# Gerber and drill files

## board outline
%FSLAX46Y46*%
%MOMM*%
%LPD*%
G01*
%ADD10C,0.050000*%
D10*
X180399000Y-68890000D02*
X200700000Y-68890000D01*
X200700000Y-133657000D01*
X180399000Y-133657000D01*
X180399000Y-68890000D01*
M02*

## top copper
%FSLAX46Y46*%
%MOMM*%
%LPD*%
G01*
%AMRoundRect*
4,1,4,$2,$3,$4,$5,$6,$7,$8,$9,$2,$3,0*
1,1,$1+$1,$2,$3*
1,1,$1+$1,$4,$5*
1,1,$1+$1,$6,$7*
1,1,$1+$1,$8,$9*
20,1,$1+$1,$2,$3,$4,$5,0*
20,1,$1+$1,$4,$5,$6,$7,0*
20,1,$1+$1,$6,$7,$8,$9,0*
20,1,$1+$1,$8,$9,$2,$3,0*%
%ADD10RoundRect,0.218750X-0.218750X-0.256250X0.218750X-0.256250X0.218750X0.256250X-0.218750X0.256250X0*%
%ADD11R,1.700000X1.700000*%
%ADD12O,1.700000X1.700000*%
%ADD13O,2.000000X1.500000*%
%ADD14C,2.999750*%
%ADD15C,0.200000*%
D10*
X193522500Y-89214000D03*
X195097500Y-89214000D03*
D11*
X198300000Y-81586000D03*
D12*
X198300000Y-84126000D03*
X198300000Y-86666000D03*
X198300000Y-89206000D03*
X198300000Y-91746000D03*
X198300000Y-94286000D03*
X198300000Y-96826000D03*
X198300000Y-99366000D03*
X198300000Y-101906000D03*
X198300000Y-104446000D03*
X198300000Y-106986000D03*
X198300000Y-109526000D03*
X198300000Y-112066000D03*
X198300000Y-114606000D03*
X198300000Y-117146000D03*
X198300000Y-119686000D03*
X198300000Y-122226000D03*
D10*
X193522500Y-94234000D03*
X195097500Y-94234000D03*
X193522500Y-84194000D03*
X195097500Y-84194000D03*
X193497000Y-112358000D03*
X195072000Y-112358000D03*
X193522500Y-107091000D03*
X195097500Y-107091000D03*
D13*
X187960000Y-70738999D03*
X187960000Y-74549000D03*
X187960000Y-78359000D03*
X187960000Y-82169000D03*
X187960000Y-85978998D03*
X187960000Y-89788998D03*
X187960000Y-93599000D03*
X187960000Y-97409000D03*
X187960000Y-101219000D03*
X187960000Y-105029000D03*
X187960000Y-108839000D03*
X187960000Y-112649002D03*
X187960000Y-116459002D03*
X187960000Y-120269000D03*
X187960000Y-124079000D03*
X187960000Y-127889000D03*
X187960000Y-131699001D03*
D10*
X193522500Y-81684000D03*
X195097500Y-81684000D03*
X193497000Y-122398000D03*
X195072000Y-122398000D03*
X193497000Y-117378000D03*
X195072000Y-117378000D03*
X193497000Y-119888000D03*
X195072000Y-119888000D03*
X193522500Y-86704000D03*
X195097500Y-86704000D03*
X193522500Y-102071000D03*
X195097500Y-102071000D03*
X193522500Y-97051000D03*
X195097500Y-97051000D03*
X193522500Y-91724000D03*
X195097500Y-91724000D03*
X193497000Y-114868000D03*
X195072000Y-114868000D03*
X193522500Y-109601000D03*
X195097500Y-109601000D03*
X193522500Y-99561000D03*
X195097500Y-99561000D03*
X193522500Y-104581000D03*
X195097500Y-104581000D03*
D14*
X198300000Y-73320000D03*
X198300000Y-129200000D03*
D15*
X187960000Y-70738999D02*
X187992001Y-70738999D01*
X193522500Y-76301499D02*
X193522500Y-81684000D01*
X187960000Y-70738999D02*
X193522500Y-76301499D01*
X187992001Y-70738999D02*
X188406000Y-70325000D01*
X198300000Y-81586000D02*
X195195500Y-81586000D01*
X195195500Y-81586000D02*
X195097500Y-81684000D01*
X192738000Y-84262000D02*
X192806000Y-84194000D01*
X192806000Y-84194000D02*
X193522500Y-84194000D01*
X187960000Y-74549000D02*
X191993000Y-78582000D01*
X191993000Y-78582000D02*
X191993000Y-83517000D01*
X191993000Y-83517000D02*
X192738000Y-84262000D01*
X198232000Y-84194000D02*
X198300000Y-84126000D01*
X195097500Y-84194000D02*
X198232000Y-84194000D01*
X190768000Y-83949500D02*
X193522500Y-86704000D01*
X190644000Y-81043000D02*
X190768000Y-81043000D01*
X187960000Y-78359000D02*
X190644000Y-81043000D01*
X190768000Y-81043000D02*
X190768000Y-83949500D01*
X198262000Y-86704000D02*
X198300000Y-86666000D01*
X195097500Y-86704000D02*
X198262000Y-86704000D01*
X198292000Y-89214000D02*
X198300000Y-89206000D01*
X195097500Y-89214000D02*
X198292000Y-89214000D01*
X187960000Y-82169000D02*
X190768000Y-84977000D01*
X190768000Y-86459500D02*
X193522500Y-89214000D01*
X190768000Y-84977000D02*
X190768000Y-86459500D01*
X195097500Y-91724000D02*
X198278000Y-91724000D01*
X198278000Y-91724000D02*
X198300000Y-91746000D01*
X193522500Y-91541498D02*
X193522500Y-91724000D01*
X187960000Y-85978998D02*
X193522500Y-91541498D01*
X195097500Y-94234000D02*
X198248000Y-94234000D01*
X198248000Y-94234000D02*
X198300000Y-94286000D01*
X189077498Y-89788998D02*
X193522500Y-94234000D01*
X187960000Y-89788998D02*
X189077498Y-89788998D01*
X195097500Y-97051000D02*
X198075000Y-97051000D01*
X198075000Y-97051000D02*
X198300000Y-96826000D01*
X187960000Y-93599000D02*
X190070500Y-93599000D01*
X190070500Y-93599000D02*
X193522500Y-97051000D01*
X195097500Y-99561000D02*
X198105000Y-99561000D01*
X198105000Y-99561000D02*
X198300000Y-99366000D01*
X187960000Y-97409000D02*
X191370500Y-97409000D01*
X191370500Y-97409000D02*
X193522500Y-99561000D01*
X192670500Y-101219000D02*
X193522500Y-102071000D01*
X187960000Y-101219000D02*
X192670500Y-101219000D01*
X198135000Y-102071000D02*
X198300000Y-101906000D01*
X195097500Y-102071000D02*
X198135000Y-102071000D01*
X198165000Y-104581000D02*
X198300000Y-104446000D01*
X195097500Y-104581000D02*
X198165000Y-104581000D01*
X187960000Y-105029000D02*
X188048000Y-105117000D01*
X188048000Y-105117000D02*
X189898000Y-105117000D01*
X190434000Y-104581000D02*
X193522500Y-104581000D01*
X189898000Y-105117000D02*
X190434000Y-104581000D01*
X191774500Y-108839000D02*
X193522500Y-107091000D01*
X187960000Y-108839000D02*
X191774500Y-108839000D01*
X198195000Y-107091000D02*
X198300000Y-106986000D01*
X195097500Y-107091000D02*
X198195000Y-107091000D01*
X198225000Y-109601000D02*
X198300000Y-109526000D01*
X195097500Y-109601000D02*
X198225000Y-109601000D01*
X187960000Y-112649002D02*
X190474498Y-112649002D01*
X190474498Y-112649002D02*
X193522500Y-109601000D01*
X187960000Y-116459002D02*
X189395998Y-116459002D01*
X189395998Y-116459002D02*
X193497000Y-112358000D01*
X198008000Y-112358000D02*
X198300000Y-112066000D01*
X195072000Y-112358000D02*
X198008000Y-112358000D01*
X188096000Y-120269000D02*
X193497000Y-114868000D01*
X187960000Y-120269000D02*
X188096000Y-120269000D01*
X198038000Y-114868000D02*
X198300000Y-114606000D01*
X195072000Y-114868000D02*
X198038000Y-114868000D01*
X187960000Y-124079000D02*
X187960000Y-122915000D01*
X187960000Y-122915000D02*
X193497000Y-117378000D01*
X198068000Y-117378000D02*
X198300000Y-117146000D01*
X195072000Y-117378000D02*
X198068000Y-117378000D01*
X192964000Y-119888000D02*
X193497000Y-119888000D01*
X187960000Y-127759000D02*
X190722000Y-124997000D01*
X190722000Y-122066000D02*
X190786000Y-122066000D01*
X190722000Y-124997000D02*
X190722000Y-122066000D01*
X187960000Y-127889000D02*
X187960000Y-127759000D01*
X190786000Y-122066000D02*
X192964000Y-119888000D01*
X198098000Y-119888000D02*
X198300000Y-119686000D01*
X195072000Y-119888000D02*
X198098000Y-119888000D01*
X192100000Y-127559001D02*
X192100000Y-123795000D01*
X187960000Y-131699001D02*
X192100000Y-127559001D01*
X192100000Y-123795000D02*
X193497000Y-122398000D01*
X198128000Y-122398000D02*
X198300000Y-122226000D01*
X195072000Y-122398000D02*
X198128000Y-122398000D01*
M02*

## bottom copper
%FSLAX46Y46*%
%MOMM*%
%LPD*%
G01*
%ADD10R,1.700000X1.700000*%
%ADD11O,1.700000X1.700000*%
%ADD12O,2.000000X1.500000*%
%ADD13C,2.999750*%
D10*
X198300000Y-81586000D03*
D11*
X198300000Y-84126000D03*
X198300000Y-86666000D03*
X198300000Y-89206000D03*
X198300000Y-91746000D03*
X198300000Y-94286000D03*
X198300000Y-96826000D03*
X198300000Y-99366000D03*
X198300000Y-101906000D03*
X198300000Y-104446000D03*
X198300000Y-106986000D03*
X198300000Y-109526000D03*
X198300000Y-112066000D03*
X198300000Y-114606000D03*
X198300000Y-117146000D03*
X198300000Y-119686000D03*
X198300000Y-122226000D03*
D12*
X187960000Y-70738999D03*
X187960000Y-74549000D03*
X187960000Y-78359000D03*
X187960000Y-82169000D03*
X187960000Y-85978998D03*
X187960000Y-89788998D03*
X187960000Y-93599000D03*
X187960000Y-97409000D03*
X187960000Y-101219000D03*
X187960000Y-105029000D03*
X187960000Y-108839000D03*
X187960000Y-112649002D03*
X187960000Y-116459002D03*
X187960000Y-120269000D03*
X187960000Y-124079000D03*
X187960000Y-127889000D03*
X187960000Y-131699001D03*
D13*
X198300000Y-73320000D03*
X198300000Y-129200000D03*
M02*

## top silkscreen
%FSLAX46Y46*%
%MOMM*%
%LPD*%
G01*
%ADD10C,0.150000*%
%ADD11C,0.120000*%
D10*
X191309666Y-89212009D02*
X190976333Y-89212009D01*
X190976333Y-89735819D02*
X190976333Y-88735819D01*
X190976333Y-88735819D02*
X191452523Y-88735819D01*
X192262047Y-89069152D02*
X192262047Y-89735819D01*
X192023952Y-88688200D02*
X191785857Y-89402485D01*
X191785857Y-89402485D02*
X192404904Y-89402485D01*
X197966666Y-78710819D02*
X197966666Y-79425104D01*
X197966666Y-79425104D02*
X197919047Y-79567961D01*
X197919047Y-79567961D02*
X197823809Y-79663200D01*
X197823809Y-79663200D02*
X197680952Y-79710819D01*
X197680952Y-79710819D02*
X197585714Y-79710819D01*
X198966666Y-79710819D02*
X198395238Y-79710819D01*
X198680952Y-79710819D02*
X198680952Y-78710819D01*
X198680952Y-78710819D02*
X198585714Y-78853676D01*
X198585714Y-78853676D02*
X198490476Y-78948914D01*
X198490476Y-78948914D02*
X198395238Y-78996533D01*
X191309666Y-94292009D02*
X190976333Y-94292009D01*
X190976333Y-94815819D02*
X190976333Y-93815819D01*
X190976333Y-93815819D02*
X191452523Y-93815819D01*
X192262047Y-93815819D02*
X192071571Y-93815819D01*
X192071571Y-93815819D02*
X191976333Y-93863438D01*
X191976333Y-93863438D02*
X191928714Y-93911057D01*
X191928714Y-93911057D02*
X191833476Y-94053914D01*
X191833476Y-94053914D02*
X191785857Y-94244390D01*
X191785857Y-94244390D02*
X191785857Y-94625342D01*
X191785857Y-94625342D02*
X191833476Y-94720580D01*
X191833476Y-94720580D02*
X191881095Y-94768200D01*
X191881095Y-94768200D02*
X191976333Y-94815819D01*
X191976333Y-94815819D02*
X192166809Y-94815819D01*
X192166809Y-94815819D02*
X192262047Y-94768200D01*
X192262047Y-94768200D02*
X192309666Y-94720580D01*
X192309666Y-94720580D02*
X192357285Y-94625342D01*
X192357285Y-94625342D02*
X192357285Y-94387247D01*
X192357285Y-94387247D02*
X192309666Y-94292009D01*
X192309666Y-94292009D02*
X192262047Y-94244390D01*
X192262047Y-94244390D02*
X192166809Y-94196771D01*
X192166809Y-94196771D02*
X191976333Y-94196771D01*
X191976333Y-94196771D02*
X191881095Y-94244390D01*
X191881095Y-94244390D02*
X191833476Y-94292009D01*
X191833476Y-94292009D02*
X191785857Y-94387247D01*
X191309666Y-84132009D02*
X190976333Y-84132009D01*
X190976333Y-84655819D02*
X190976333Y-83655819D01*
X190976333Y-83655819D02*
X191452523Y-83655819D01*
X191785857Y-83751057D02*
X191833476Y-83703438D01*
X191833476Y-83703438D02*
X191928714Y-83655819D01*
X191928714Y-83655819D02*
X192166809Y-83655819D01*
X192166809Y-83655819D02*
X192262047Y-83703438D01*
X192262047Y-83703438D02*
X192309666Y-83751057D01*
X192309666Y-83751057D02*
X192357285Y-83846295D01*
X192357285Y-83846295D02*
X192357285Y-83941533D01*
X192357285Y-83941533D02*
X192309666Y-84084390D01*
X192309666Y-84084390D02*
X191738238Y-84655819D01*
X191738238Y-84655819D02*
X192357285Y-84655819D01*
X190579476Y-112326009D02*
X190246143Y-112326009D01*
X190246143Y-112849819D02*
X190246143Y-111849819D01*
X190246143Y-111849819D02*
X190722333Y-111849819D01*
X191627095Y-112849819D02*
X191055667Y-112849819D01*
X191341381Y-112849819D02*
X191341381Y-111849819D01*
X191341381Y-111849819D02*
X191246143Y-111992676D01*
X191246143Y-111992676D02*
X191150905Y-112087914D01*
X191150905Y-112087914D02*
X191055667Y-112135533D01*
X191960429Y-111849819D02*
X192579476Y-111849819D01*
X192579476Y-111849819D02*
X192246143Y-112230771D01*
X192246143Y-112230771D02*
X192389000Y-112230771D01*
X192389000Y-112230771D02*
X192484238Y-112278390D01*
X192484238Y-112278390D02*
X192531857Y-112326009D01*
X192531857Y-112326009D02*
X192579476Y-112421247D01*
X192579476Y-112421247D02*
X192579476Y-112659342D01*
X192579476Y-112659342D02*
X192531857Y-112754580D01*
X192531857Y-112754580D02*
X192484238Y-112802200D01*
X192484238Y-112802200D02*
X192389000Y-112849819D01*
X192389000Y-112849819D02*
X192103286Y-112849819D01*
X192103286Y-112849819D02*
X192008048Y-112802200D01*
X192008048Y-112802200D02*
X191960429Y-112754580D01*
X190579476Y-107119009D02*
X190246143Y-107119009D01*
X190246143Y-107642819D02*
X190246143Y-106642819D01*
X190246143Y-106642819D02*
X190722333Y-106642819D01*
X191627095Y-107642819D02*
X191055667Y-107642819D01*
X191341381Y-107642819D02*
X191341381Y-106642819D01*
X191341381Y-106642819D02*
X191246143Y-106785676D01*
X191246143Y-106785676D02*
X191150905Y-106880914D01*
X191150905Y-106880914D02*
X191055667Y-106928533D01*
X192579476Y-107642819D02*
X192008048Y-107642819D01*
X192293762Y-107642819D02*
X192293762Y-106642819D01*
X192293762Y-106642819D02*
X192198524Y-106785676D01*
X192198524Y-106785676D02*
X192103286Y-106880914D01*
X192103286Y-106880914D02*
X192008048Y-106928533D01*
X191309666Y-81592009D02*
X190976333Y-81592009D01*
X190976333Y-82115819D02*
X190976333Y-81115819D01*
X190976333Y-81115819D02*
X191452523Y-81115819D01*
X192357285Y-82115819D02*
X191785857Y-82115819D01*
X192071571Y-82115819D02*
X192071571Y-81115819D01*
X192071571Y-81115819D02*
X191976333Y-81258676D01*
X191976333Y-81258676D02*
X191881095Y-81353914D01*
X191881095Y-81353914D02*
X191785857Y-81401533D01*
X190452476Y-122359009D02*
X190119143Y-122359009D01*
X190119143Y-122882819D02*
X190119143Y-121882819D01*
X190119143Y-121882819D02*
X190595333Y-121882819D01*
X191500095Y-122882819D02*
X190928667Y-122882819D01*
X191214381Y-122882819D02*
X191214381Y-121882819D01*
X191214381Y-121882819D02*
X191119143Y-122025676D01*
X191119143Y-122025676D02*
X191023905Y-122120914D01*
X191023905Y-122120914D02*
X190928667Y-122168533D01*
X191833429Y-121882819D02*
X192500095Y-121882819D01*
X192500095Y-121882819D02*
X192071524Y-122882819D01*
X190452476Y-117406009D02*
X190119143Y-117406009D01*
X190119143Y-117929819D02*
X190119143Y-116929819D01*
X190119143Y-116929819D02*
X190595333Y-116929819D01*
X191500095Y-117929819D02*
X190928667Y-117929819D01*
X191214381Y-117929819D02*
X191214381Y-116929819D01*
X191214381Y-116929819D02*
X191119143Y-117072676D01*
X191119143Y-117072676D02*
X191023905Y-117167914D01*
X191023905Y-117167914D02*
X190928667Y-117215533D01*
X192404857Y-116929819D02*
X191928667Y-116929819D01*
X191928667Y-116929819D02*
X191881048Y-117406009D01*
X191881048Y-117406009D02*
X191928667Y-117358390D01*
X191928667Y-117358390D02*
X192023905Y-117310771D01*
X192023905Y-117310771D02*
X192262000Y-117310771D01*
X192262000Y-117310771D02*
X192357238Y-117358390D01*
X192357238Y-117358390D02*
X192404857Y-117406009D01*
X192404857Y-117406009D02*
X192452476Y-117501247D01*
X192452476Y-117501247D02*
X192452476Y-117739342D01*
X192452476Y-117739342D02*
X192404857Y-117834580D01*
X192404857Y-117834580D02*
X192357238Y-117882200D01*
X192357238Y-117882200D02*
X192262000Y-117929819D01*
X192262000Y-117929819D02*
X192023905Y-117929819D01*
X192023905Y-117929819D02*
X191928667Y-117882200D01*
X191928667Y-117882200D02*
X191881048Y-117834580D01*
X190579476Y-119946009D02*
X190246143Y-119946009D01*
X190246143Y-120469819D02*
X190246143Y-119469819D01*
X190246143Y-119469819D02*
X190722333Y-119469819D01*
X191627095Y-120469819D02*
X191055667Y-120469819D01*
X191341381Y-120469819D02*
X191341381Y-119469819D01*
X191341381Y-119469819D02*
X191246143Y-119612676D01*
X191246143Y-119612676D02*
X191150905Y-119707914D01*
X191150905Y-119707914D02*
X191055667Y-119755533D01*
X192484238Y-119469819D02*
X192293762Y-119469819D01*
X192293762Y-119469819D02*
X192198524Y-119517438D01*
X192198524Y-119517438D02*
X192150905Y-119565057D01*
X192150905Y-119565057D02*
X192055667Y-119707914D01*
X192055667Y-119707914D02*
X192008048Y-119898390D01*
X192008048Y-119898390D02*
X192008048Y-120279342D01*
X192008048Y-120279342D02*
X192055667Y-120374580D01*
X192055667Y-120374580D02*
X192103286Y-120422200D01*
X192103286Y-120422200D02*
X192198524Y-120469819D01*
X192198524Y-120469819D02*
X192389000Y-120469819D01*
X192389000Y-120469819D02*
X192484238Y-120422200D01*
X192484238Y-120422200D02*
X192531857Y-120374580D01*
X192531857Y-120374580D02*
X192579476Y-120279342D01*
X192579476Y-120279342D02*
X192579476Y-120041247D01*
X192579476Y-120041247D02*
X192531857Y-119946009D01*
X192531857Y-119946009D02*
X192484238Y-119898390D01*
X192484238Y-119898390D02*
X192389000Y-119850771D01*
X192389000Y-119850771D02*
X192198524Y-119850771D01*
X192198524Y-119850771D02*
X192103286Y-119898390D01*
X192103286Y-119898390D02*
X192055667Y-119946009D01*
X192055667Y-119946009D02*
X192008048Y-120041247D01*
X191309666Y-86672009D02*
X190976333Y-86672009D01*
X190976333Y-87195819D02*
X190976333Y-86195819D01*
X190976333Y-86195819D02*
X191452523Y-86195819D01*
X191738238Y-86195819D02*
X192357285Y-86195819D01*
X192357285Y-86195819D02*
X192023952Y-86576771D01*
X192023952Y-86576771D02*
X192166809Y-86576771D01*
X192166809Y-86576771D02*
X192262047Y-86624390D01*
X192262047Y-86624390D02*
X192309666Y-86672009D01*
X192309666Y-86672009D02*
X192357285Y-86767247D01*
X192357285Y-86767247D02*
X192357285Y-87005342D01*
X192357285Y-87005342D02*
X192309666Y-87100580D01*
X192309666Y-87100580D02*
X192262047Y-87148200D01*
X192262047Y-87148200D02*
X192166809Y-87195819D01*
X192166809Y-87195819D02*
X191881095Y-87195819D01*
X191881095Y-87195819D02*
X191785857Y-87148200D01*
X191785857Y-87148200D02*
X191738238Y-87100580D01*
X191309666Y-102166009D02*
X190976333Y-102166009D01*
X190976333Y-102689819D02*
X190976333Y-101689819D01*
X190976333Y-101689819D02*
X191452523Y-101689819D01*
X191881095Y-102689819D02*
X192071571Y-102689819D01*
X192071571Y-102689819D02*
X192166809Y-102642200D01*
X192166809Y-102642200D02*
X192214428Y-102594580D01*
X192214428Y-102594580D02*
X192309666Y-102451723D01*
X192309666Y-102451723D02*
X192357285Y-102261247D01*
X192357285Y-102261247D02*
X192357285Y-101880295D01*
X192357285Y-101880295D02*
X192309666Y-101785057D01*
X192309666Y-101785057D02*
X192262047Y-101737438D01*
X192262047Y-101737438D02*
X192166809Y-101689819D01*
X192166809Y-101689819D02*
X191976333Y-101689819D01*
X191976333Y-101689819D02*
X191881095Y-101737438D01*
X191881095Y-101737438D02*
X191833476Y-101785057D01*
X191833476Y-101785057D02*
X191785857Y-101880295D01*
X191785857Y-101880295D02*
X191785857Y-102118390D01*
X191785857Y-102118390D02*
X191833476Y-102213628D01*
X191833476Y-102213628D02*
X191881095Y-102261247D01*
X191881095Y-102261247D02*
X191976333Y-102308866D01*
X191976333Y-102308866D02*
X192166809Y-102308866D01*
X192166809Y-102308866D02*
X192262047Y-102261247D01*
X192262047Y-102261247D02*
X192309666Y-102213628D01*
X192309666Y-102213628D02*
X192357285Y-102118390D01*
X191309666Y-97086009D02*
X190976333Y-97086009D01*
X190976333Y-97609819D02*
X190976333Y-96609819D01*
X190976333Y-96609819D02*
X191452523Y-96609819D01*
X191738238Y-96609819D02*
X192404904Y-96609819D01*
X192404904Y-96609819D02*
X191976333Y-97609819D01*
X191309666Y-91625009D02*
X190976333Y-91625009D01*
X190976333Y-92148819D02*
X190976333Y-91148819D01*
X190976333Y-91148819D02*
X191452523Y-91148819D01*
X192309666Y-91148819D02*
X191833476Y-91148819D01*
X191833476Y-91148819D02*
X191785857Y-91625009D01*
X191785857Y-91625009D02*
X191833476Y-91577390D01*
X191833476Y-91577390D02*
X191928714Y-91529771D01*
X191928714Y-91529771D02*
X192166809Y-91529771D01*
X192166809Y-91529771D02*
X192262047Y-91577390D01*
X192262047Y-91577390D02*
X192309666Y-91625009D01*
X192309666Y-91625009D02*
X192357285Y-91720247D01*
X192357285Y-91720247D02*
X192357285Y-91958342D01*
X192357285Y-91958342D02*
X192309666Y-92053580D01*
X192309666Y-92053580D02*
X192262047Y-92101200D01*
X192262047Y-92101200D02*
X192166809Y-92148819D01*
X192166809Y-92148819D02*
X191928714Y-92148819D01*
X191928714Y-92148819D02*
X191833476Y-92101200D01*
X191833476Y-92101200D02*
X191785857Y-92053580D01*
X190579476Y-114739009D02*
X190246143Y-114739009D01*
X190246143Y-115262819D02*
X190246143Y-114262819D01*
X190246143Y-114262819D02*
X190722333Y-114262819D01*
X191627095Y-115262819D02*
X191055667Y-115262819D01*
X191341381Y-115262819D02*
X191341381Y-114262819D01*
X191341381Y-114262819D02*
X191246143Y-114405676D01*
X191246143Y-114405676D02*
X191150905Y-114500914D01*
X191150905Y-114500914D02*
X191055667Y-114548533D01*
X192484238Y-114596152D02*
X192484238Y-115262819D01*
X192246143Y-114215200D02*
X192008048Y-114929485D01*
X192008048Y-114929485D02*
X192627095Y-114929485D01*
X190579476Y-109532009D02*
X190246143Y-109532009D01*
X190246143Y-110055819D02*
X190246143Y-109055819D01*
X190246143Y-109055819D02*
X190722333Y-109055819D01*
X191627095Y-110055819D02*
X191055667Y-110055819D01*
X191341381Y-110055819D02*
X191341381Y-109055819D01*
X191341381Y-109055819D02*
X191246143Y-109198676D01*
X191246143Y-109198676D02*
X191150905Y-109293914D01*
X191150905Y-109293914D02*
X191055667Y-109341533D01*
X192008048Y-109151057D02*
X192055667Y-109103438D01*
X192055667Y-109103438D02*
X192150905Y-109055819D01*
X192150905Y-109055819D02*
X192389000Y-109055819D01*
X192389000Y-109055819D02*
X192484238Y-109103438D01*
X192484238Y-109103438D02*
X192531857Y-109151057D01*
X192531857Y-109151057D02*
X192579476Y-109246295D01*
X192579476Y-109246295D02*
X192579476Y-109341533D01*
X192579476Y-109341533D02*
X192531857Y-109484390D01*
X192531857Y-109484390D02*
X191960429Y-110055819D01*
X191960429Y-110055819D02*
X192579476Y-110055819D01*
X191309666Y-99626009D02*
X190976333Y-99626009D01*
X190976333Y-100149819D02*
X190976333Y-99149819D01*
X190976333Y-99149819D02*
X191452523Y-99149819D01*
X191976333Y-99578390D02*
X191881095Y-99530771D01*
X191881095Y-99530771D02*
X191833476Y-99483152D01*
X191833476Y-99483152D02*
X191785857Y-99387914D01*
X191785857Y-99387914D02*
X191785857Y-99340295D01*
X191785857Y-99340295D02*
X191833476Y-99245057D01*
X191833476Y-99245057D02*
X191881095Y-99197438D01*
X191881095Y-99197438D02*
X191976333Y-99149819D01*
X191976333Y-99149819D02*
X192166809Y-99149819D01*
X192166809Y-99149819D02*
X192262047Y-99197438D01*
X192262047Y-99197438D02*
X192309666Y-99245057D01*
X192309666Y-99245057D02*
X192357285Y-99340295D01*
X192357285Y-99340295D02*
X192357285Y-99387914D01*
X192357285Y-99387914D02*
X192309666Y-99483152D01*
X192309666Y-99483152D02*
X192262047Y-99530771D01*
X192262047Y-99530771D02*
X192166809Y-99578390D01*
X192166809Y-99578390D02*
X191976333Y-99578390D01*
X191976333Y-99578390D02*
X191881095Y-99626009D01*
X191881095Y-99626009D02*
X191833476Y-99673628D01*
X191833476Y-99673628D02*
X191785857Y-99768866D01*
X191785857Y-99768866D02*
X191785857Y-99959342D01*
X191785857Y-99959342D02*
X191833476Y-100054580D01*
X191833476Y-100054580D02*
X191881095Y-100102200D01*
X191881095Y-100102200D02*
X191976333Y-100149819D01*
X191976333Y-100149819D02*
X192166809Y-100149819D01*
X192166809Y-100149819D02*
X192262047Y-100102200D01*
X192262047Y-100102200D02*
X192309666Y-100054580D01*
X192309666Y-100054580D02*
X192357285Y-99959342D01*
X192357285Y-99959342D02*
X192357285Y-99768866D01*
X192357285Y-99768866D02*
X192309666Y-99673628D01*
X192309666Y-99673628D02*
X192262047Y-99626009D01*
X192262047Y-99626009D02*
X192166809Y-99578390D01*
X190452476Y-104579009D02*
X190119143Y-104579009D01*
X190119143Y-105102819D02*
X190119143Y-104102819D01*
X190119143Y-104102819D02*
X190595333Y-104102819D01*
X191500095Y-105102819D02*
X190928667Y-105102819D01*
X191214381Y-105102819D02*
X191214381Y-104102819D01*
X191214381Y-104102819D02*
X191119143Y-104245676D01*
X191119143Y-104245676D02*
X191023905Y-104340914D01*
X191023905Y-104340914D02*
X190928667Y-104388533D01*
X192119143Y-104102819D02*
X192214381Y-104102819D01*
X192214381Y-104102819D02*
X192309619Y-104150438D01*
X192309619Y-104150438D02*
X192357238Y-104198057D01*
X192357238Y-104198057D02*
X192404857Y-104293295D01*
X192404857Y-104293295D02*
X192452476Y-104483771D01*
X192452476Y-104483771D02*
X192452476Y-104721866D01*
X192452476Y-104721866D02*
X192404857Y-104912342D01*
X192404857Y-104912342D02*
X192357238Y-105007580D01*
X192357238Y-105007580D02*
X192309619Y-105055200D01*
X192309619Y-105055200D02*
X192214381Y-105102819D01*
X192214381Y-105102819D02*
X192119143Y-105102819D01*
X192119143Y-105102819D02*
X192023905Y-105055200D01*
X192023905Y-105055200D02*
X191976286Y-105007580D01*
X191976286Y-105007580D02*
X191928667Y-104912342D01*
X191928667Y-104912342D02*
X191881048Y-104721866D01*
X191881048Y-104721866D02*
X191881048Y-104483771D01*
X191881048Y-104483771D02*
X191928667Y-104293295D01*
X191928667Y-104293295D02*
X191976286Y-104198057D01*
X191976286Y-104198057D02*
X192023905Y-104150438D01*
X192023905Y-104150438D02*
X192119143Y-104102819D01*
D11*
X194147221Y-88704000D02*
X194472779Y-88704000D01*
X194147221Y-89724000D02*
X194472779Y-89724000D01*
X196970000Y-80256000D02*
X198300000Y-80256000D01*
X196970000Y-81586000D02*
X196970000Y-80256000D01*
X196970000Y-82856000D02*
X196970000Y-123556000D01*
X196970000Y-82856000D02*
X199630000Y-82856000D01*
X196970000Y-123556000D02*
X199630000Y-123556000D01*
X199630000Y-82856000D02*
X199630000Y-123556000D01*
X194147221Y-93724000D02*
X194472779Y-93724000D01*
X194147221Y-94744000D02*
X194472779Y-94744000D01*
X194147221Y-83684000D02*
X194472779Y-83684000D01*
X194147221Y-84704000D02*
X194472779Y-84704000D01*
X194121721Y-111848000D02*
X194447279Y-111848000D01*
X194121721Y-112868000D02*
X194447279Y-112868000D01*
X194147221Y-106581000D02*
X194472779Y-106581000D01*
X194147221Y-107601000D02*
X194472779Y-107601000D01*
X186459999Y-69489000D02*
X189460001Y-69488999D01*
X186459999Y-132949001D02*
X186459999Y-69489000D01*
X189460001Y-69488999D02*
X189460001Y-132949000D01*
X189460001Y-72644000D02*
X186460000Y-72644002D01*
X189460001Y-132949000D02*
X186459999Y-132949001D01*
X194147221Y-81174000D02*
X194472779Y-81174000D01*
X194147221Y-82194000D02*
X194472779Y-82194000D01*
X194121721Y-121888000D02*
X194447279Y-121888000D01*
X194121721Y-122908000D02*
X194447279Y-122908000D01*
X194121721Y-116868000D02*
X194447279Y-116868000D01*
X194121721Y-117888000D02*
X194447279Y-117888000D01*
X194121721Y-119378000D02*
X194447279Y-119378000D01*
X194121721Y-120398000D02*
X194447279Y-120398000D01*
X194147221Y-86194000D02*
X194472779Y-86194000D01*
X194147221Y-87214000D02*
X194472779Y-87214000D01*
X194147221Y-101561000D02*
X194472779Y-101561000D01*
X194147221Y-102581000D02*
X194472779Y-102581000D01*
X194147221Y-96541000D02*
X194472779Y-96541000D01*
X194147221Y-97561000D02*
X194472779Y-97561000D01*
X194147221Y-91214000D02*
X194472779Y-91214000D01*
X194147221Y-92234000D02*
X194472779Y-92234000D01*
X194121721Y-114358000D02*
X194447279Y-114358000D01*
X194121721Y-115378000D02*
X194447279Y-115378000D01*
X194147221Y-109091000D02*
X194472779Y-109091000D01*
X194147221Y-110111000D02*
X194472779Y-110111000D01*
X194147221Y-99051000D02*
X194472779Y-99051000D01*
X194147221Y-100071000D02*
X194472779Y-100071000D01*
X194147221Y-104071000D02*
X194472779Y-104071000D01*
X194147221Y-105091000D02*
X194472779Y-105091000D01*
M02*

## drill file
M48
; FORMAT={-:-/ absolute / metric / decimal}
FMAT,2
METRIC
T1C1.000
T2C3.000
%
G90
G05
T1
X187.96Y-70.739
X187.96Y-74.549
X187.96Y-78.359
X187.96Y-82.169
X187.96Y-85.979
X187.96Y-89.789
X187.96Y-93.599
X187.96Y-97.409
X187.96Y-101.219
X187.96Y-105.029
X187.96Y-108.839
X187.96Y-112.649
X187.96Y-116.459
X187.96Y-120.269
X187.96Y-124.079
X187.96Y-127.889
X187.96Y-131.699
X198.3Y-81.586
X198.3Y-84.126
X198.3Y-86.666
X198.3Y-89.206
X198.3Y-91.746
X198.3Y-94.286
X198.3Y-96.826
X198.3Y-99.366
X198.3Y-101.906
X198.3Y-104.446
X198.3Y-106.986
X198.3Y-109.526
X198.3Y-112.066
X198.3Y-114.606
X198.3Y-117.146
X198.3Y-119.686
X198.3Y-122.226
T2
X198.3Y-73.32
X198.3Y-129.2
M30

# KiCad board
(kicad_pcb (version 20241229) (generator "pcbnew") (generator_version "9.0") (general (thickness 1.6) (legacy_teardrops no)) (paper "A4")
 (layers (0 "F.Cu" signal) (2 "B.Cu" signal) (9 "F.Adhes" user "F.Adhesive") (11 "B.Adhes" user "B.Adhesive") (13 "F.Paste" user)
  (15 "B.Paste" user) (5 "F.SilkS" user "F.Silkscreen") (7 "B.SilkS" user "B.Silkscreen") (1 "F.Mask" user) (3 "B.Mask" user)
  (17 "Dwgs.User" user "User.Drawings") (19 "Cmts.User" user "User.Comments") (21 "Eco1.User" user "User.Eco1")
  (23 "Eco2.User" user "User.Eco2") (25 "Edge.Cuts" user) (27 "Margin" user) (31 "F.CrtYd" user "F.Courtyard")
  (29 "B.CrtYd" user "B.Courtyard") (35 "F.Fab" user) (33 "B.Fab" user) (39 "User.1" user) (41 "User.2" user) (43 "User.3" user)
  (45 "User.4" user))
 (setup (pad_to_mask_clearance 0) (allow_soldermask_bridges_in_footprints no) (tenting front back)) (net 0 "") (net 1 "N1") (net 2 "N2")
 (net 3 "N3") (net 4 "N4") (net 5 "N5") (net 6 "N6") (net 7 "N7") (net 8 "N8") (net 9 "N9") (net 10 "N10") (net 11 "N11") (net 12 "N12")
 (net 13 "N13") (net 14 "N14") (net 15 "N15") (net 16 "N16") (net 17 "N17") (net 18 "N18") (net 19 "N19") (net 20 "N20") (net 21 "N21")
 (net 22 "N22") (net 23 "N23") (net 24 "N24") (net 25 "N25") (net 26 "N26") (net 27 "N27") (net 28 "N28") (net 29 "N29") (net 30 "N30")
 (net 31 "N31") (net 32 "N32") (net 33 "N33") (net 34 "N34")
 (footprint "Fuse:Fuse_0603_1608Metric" (layer "F.Cu") (at 194.31 89.214)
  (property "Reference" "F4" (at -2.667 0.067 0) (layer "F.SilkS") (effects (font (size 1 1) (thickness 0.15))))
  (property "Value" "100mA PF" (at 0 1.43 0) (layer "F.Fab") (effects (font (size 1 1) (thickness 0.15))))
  (fp_line (start -0.162779 -0.51) (end 0.162779 -0.51) (stroke (width 0.12) (type solid)) (layer "F.SilkS"))
  (fp_line (start -0.162779 0.51) (end 0.162779 0.51) (stroke (width 0.12) (type solid)) (layer "F.SilkS"))
  (pad "1" smd roundrect (at -0.7875 0) (size 0.875 0.95) (layers "F.Cu" "F.Mask" "F.Paste") (roundrect_rratio 0.25) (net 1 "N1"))
  (pad "2" smd roundrect (at 0.7875 0) (size 0.875 0.95) (layers "F.Cu" "F.Mask" "F.Paste") (roundrect_rratio 0.25) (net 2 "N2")))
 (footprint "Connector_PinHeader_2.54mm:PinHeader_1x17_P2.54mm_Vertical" (layer "F.Cu") (at 198.3 81.586)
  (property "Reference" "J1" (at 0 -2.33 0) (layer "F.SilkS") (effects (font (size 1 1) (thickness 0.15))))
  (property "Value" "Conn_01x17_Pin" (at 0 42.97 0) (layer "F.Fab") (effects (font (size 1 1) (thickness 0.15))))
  (fp_line (start -1.33 -1.33) (end 0 -1.33) (stroke (width 0.12) (type solid)) (layer "F.SilkS"))
  (fp_line (start -1.33 0) (end -1.33 -1.33) (stroke (width 0.12) (type solid)) (layer "F.SilkS"))
  (fp_line (start -1.33 1.27) (end -1.33 41.97) (stroke (width 0.12) (type solid)) (layer "F.SilkS"))
  (fp_line (start -1.33 1.27) (end 1.33 1.27) (stroke (width 0.12) (type solid)) (layer "F.SilkS"))
  (fp_line (start -1.33 41.97) (end 1.33 41.97) (stroke (width 0.12) (type solid)) (layer "F.SilkS"))
  (fp_line (start 1.33 1.27) (end 1.33 41.97) (stroke (width 0.12) (type solid)) (layer "F.SilkS"))
  (pad "1" thru_hole rect (at 0 0) (size 1.7 1.7) (drill 1) (layers "*.Cu" "*.Mask") (remove_unused_layers no) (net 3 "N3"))
  (pad "2" thru_hole oval (at 0 2.54) (size 1.7 1.7) (drill 1) (layers "*.Cu" "*.Mask") (remove_unused_layers no) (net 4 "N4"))
  (pad "3" thru_hole oval (at 0 5.08) (size 1.7 1.7) (drill 1) (layers "*.Cu" "*.Mask") (remove_unused_layers no) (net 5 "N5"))
  (pad "4" thru_hole oval (at 0 7.62) (size 1.7 1.7) (drill 1) (layers "*.Cu" "*.Mask") (remove_unused_layers no) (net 2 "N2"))
  (pad "5" thru_hole oval (at 0 10.16) (size 1.7 1.7) (drill 1) (layers "*.Cu" "*.Mask") (remove_unused_layers no) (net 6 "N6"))
  (pad "6" thru_hole oval (at 0 12.7) (size 1.7 1.7) (drill 1) (layers "*.Cu" "*.Mask") (remove_unused_layers no) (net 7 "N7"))
  (pad "7" thru_hole oval (at 0 15.24) (size 1.7 1.7) (drill 1) (layers "*.Cu" "*.Mask") (remove_unused_layers no) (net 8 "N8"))
  (pad "8" thru_hole oval (at 0 17.78) (size 1.7 1.7) (drill 1) (layers "*.Cu" "*.Mask") (remove_unused_layers no) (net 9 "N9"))
  (pad "9" thru_hole oval (at 0 20.32) (size 1.7 1.7) (drill 1) (layers "*.Cu" "*.Mask") (remove_unused_layers no) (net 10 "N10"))
  (pad "10" thru_hole oval (at 0 22.86) (size 1.7 1.7) (drill 1) (layers "*.Cu" "*.Mask") (remove_unused_layers no) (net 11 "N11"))
  (pad "11" thru_hole oval (at 0 25.4) (size 1.7 1.7) (drill 1) (layers "*.Cu" "*.Mask") (remove_unused_layers no) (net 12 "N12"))
  (pad "12" thru_hole oval (at 0 27.94) (size 1.7 1.7) (drill 1) (layers "*.Cu" "*.Mask") (remove_unused_layers no) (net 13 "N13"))
  (pad "13" thru_hole oval (at 0 30.48) (size 1.7 1.7) (drill 1) (layers "*.Cu" "*.Mask") (remove_unused_layers no) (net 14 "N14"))
  (pad "14" thru_hole oval (at 0 33.02) (size 1.7 1.7) (drill 1) (layers "*.Cu" "*.Mask") (remove_unused_layers no) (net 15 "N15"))
  (pad "15" thru_hole oval (at 0 35.56) (size 1.7 1.7) (drill 1) (layers "*.Cu" "*.Mask") (remove_unused_layers no) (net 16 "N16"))
  (pad "16" thru_hole oval (at 0 38.1) (size 1.7 1.7) (drill 1) (layers "*.Cu" "*.Mask") (remove_unused_layers no) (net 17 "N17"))
  (pad "17" thru_hole oval (at 0 40.64) (size 1.7 1.7) (drill 1) (layers "*.Cu" "*.Mask") (remove_unused_layers no) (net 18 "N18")))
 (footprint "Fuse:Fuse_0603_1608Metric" (layer "F.Cu") (at 194.31 94.234)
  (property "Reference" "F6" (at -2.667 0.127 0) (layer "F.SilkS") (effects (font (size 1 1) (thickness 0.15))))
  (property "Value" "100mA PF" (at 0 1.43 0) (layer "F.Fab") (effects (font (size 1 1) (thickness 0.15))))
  (fp_line (start -0.162779 -0.51) (end 0.162779 -0.51) (stroke (width 0.12) (type solid)) (layer "F.SilkS"))
  (fp_line (start -0.162779 0.51) (end 0.162779 0.51) (stroke (width 0.12) (type solid)) (layer "F.SilkS"))
  (pad "1" smd roundrect (at -0.7875 0) (size 0.875 0.95) (layers "F.Cu" "F.Mask" "F.Paste") (roundrect_rratio 0.25) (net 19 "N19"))
  (pad "2" smd roundrect (at 0.7875 0) (size 0.875 0.95) (layers "F.Cu" "F.Mask" "F.Paste") (roundrect_rratio 0.25) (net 7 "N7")))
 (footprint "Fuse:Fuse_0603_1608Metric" (layer "F.Cu") (at 194.31 84.194)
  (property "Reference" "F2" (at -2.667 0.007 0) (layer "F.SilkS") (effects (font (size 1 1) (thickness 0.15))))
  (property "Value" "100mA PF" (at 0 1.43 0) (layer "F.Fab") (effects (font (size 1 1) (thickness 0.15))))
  (fp_line (start -0.162779 -0.51) (end 0.162779 -0.51) (stroke (width 0.12) (type solid)) (layer "F.SilkS"))
  (fp_line (start -0.162779 0.51) (end 0.162779 0.51) (stroke (width 0.12) (type solid)) (layer "F.SilkS"))
  (pad "1" smd roundrect (at -0.7875 0) (size 0.875 0.95) (layers "F.Cu" "F.Mask" "F.Paste") (roundrect_rratio 0.25) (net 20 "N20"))
  (pad "2" smd roundrect (at 0.7875 0) (size 0.875 0.95) (layers "F.Cu" "F.Mask" "F.Paste") (roundrect_rratio 0.25) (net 4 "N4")))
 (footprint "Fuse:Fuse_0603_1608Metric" (layer "F.Cu") (at 194.2845 112.358)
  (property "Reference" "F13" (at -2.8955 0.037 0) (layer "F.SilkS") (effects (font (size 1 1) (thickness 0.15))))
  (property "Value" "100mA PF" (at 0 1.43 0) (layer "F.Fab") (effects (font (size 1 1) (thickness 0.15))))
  (fp_line (start -0.162779 -0.51) (end 0.162779 -0.51) (stroke (width 0.12) (type solid)) (layer "F.SilkS"))
  (fp_line (start -0.162779 0.51) (end 0.162779 0.51) (stroke (width 0.12) (type solid)) (layer "F.SilkS"))
  (pad "1" smd roundrect (at -0.7875 0) (size 0.875 0.95) (layers "F.Cu" "F.Mask" "F.Paste") (roundrect_rratio 0.25) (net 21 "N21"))
  (pad "2" smd roundrect (at 0.7875 0) (size 0.875 0.95) (layers "F.Cu" "F.Mask" "F.Paste") (roundrect_rratio 0.25) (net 14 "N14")))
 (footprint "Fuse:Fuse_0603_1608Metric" (layer "F.Cu") (at 194.31 107.091)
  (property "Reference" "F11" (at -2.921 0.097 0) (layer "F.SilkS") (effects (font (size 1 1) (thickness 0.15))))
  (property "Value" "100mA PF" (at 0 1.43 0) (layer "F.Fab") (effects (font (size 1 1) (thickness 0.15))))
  (fp_line (start -0.162779 -0.51) (end 0.162779 -0.51) (stroke (width 0.12) (type solid)) (layer "F.SilkS"))
  (fp_line (start -0.162779 0.51) (end 0.162779 0.51) (stroke (width 0.12) (type solid)) (layer "F.SilkS"))
  (pad "1" smd roundrect (at -0.7875 0) (size 0.875 0.95) (layers "F.Cu" "F.Mask" "F.Paste") (roundrect_rratio 0.25) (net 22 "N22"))
  (pad "2" smd roundrect (at 0.7875 0) (size 0.875 0.95) (layers "F.Cu" "F.Mask" "F.Paste") (roundrect_rratio 0.25) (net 12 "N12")))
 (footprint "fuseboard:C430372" (layer "F.Cu") (at 187.96 101.219 -90)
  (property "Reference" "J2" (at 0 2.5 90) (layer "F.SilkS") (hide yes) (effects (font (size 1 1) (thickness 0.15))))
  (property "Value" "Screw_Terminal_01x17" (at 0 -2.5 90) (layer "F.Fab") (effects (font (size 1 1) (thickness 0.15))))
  (fp_line (start -31.73 1.500001) (end -31.730001 -1.500001) (stroke (width 0.12) (type default)) (layer "F.SilkS"))
  (fp_line (start 31.730001 1.500001) (end -31.73 1.500001) (stroke (width 0.12) (type default)) (layer "F.SilkS"))
  (fp_line (start -31.730001 -1.500001) (end 31.73 -1.500001) (stroke (width 0.12) (type default)) (layer "F.SilkS"))
  (fp_line (start -28.575 -1.500001) (end -28.574998 1.5) (stroke (width 0.12) (type default)) (layer "F.SilkS"))
  (fp_line (start 31.73 -1.500001) (end 31.730001 1.500001) (stroke (width 0.12) (type default)) (layer "F.SilkS"))
  (pad "1" thru_hole oval (at -30.480001 0 270) (size 1.5 2) (drill 1) (layers "*.Cu" "*.Mask") (remove_unused_layers no) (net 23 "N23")
   (thermal_bridge_angle 45))
  (pad "2" thru_hole oval (at -26.67 0 270) (size 1.5 2) (drill 1) (layers "*.Cu" "*.Mask") (remove_unused_layers no) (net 20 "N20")
   (thermal_bridge_angle 45))
  (pad "3" thru_hole oval (at -22.86 0 270) (size 1.5 2) (drill 1) (layers "*.Cu" "*.Mask") (remove_unused_layers no) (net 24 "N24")
   (thermal_bridge_angle 45))
  (pad "4" thru_hole oval (at -19.05 0 270) (size 1.5 2) (drill 1) (layers "*.Cu" "*.Mask") (remove_unused_layers no) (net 1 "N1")
   (thermal_bridge_angle 45))
  (pad "5" thru_hole oval (at -15.240002 0 270) (size 1.5 2) (drill 1) (layers "*.Cu" "*.Mask") (remove_unused_layers no) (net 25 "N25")
   (thermal_bridge_angle 45))
  (pad "6" thru_hole oval (at -11.430002 0 270) (size 1.5 2) (drill 1) (layers "*.Cu" "*.Mask") (remove_unused_layers no) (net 19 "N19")
   (thermal_bridge_angle 45))
  (pad "7" thru_hole oval (at -7.62 0 270) (size 1.5 2) (drill 1) (layers "*.Cu" "*.Mask") (remove_unused_layers no) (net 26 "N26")
   (thermal_bridge_angle 45))
  (pad "8" thru_hole oval (at -3.81 0 270) (size 1.5 2) (drill 1) (layers "*.Cu" "*.Mask") (remove_unused_layers no) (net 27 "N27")
   (thermal_bridge_angle 45))
  (pad "9" thru_hole oval (at 0 0 270) (size 1.5 2) (drill 1) (layers "*.Cu" "*.Mask") (remove_unused_layers no) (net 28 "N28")
   (thermal_bridge_angle 45))
  (pad "10" thru_hole oval (at 3.81 0 270) (size 1.5 2) (drill 1) (layers "*.Cu" "*.Mask") (remove_unused_layers no) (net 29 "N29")
   (thermal_bridge_angle 45))
  (pad "11" thru_hole oval (at 7.62 0 270) (size 1.5 2) (drill 1) (layers "*.Cu" "*.Mask") (remove_unused_layers no) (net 22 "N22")
   (thermal_bridge_angle 45))
  (pad "12" thru_hole oval (at 11.430002 0 270) (size 1.5 2) (drill 1) (layers "*.Cu" "*.Mask") (remove_unused_layers no) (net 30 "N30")
   (thermal_bridge_angle 45))
  (pad "13" thru_hole oval (at 15.240002 0 270) (size 1.5 2) (drill 1) (layers "*.Cu" "*.Mask") (remove_unused_layers no) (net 21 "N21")
   (thermal_bridge_angle 45))
  (pad "14" thru_hole oval (at 19.05 0 270) (size 1.5 2) (drill 1) (layers "*.Cu" "*.Mask") (remove_unused_layers no) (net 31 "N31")
   (thermal_bridge_angle 45))
  (pad "15" thru_hole oval (at 22.86 0 270) (size 1.5 2) (drill 1) (layers "*.Cu" "*.Mask") (remove_unused_layers no) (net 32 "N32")
   (thermal_bridge_angle 45))
  (pad "16" thru_hole oval (at 26.67 0 270) (size 1.5 2) (drill 1) (layers "*.Cu" "*.Mask") (remove_unused_layers no) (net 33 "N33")
   (thermal_bridge_angle 45))
  (pad "17" thru_hole oval (at 30.480001 0 270) (size 1.5 2) (drill 1) (layers "*.Cu" "*.Mask") (remove_unused_layers no) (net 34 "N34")
   (thermal_bridge_angle 45)))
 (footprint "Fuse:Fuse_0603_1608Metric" (layer "F.Cu") (at 194.31 81.684)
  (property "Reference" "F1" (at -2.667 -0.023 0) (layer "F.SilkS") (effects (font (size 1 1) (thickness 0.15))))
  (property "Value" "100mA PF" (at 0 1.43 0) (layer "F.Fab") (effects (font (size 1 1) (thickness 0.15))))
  (fp_line (start -0.162779 -0.51) (end 0.162779 -0.51) (stroke (width 0.12) (type solid)) (layer "F.SilkS"))
  (fp_line (start -0.162779 0.51) (end 0.162779 0.51) (stroke (width 0.12) (type solid)) (layer "F.SilkS"))
  (pad "1" smd roundrect (at -0.7875 0) (size 0.875 0.95) (layers "F.Cu" "F.Mask" "F.Paste") (roundrect_rratio 0.25) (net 23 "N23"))
  (pad "2" smd roundrect (at 0.7875 0) (size 0.875 0.95) (layers "F.Cu" "F.Mask" "F.Paste") (roundrect_rratio 0.25) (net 3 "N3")))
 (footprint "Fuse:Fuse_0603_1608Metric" (layer "F.Cu") (at 194.2845 122.398)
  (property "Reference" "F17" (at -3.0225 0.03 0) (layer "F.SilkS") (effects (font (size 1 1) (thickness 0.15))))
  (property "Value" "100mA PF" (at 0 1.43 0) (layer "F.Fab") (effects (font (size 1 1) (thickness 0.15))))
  (fp_line (start -0.162779 -0.51) (end 0.162779 -0.51) (stroke (width 0.12) (type solid)) (layer "F.SilkS"))
  (fp_line (start -0.162779 0.51) (end 0.162779 0.51) (stroke (width 0.12) (type solid)) (layer "F.SilkS"))
  (pad "1" smd roundrect (at -0.7875 0) (size 0.875 0.95) (layers "F.Cu" "F.Mask" "F.Paste") (roundrect_rratio 0.25) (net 34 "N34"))
  (pad "2" smd roundrect (at 0.7875 0) (size 0.875 0.95) (layers "F.Cu" "F.Mask" "F.Paste") (roundrect_rratio 0.25) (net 18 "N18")))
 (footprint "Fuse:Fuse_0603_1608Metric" (layer "F.Cu") (at 194.2845 117.378)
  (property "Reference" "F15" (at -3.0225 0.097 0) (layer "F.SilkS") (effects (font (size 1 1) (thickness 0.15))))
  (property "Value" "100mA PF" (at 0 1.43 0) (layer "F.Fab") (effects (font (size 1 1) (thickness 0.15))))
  (fp_line (start -0.162779 -0.51) (end 0.162779 -0.51) (stroke (width 0.12) (type solid)) (layer "F.SilkS"))
  (fp_line (start -0.162779 0.51) (end 0.162779 0.51) (stroke (width 0.12) (type solid)) (layer "F.SilkS"))
  (pad "1" smd roundrect (at -0.7875 0) (size 0.875 0.95) (layers "F.Cu" "F.Mask" "F.Paste") (roundrect_rratio 0.25) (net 32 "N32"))
  (pad "2" smd roundrect (at 0.7875 0) (size 0.875 0.95) (layers "F.Cu" "F.Mask" "F.Paste") (roundrect_rratio 0.25) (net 16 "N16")))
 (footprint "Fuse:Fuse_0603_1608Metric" (layer "F.Cu") (at 194.2845 119.888)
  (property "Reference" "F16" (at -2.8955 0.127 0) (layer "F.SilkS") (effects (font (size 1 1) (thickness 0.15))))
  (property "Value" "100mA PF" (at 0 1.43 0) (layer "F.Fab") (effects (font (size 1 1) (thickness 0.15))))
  (fp_line (start -0.162779 -0.51) (end 0.162779 -0.51) (stroke (width 0.12) (type solid)) (layer "F.SilkS"))
  (fp_line (start -0.162779 0.51) (end 0.162779 0.51) (stroke (width 0.12) (type solid)) (layer "F.SilkS"))
  (pad "1" smd roundrect (at -0.7875 0) (size 0.875 0.95) (layers "F.Cu" "F.Mask" "F.Paste") (roundrect_rratio 0.25) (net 33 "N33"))
  (pad "2" smd roundrect (at 0.7875 0) (size 0.875 0.95) (layers "F.Cu" "F.Mask" "F.Paste") (roundrect_rratio 0.25) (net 17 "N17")))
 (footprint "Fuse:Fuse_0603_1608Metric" (layer "F.Cu") (at 194.31 86.704)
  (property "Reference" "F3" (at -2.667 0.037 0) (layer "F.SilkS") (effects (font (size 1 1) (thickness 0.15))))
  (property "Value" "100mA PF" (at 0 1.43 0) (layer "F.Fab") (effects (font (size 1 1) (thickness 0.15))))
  (fp_line (start -0.162779 -0.51) (end 0.162779 -0.51) (stroke (width 0.12) (type solid)) (layer "F.SilkS"))
  (fp_line (start -0.162779 0.51) (end 0.162779 0.51) (stroke (width 0.12) (type solid)) (layer "F.SilkS"))
  (pad "1" smd roundrect (at -0.7875 0) (size 0.875 0.95) (layers "F.Cu" "F.Mask" "F.Paste") (roundrect_rratio 0.25) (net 24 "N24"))
  (pad "2" smd roundrect (at 0.7875 0) (size 0.875 0.95) (layers "F.Cu" "F.Mask" "F.Paste") (roundrect_rratio 0.25) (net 5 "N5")))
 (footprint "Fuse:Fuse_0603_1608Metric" (layer "F.Cu") (at 194.31 102.071)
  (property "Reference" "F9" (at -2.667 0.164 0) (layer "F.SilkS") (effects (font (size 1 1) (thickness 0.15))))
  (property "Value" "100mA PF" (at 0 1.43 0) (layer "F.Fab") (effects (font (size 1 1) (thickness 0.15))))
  (fp_line (start -0.162779 -0.51) (end 0.162779 -0.51) (stroke (width 0.12) (type solid)) (layer "F.SilkS"))
  (fp_line (start -0.162779 0.51) (end 0.162779 0.51) (stroke (width 0.12) (type solid)) (layer "F.SilkS"))
  (pad "1" smd roundrect (at -0.7875 0) (size 0.875 0.95) (layers "F.Cu" "F.Mask" "F.Paste") (roundrect_rratio 0.25) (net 28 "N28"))
  (pad "2" smd roundrect (at 0.7875 0) (size 0.875 0.95) (layers "F.Cu" "F.Mask" "F.Paste") (roundrect_rratio 0.25) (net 10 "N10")))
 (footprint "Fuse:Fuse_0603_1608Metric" (layer "F.Cu") (at 194.31 97.051)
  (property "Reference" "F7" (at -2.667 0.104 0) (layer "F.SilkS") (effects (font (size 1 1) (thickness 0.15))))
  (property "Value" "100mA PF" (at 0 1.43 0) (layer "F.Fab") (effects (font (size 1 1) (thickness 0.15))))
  (fp_line (start -0.162779 -0.51) (end 0.162779 -0.51) (stroke (width 0.12) (type solid)) (layer "F.SilkS"))
  (fp_line (start -0.162779 0.51) (end 0.162779 0.51) (stroke (width 0.12) (type solid)) (layer "F.SilkS"))
  (pad "1" smd roundrect (at -0.7875 0) (size 0.875 0.95) (layers "F.Cu" "F.Mask" "F.Paste") (roundrect_rratio 0.25) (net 26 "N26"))
  (pad "2" smd roundrect (at 0.7875 0) (size 0.875 0.95) (layers "F.Cu" "F.Mask" "F.Paste") (roundrect_rratio 0.25) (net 8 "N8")))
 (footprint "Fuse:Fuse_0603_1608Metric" (layer "F.Cu") (at 194.31 91.724)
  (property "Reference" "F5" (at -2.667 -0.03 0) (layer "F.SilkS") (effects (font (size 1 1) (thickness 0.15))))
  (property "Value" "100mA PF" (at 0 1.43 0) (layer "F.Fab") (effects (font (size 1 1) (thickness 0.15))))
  (fp_line (start -0.162779 -0.51) (end 0.162779 -0.51) (stroke (width 0.12) (type solid)) (layer "F.SilkS"))
  (fp_line (start -0.162779 0.51) (end 0.162779 0.51) (stroke (width 0.12) (type solid)) (layer "F.SilkS"))
  (pad "1" smd roundrect (at -0.7875 0) (size 0.875 0.95) (layers "F.Cu" "F.Mask" "F.Paste") (roundrect_rratio 0.25) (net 25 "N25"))
  (pad "2" smd roundrect (at 0.7875 0) (size 0.875 0.95) (layers "F.Cu" "F.Mask" "F.Paste") (roundrect_rratio 0.25) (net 6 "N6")))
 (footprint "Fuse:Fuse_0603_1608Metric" (layer "F.Cu") (at 194.2845 114.868)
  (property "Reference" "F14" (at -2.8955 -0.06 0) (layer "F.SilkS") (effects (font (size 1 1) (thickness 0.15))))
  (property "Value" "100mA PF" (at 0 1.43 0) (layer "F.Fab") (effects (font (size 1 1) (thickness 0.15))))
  (fp_line (start -0.162779 -0.51) (end 0.162779 -0.51) (stroke (width 0.12) (type solid)) (layer "F.SilkS"))
  (fp_line (start -0.162779 0.51) (end 0.162779 0.51) (stroke (width 0.12) (type solid)) (layer "F.SilkS"))
  (pad "1" smd roundrect (at -0.7875 0) (size 0.875 0.95) (layers "F.Cu" "F.Mask" "F.Paste") (roundrect_rratio 0.25) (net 31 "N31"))
  (pad "2" smd roundrect (at 0.7875 0) (size 0.875 0.95) (layers "F.Cu" "F.Mask" "F.Paste") (roundrect_rratio 0.25) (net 15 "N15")))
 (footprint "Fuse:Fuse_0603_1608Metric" (layer "F.Cu") (at 194.31 109.601)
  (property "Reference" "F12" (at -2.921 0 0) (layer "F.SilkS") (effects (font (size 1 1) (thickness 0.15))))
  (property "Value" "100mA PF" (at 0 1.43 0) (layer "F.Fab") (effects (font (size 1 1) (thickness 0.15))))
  (fp_line (start -0.162779 -0.51) (end 0.162779 -0.51) (stroke (width 0.12) (type solid)) (layer "F.SilkS"))
  (fp_line (start -0.162779 0.51) (end 0.162779 0.51) (stroke (width 0.12) (type solid)) (layer "F.SilkS"))
  (pad "1" smd roundrect (at -0.7875 0) (size 0.875 0.95) (layers "F.Cu" "F.Mask" "F.Paste") (roundrect_rratio 0.25) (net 30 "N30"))
  (pad "2" smd roundrect (at 0.7875 0) (size 0.875 0.95) (layers "F.Cu" "F.Mask" "F.Paste") (roundrect_rratio 0.25) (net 13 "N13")))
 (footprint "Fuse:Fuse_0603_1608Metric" (layer "F.Cu") (at 194.31 99.561)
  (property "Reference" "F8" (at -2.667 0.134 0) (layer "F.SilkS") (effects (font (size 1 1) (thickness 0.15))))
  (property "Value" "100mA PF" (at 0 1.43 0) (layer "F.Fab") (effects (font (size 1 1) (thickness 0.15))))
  (fp_line (start -0.162779 -0.51) (end 0.162779 -0.51) (stroke (width 0.12) (type solid)) (layer "F.SilkS"))
  (fp_line (start -0.162779 0.51) (end 0.162779 0.51) (stroke (width 0.12) (type solid)) (layer "F.SilkS"))
  (pad "1" smd roundrect (at -0.7875 0) (size 0.875 0.95) (layers "F.Cu" "F.Mask" "F.Paste") (roundrect_rratio 0.25) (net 27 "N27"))
  (pad "2" smd roundrect (at 0.7875 0) (size 0.875 0.95) (layers "F.Cu" "F.Mask" "F.Paste") (roundrect_rratio 0.25) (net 9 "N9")))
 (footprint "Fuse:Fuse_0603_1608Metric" (layer "F.Cu") (at 194.31 104.581)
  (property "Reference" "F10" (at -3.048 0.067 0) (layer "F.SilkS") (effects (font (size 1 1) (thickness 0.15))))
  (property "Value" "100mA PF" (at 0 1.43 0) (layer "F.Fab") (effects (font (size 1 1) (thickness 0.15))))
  (fp_line (start -0.162779 -0.51) (end 0.162779 -0.51) (stroke (width 0.12) (type solid)) (layer "F.SilkS"))
  (fp_line (start -0.162779 0.51) (end 0.162779 0.51) (stroke (width 0.12) (type solid)) (layer "F.SilkS"))
  (pad "1" smd roundrect (at -0.7875 0) (size 0.875 0.95) (layers "F.Cu" "F.Mask" "F.Paste") (roundrect_rratio 0.25) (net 29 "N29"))
  (pad "2" smd roundrect (at 0.7875 0) (size 0.875 0.95) (layers "F.Cu" "F.Mask" "F.Paste") (roundrect_rratio 0.25) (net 11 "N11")))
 (gr_rect (start 180.399 68.89) (end 200.7 133.657) (stroke (width 0.05) (type default)) (fill no) (layer "Edge.Cuts"))
 (via (at 198.3 73.32) (size 2.99975) (drill 2.99974) (layers "F.Cu" "B.Cu") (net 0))
 (via (at 198.3 129.2) (size 2.99975) (drill 2.99974) (layers "F.Cu" "B.Cu") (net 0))
 (segment (start 187.96 70.738999) (end 187.992001 70.738999) (width 0.2) (layer "F.Cu") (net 23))
 (segment (start 193.5225 76.301499) (end 193.5225 81.684) (width 0.2) (layer "F.Cu") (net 23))
 (segment (start 187.96 70.738999) (end 193.5225 76.301499) (width 0.2) (layer "F.Cu") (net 23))
 (segment (start 187.992001 70.738999) (end 188.406 70.325) (width 0.2) (layer "F.Cu") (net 23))
 (segment (start 198.3 81.586) (end 195.1955 81.586) (width 0.2) (layer "F.Cu") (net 3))
 (segment (start 195.1955 81.586) (end 195.0975 81.684) (width 0.2) (layer "F.Cu") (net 3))
 (segment (start 192.738 84.262) (end 192.806 84.194) (width 0.2) (layer "F.Cu") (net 20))
 (segment (start 192.806 84.194) (end 193.5225 84.194) (width 0.2) (layer "F.Cu") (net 20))
 (segment (start 187.96 74.549) (end 191.993 78.582) (width 0.2) (layer "F.Cu") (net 20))
 (segment (start 191.993 78.582) (end 191.993 83.517) (width 0.2) (layer "F.Cu") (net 20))
 (segment (start 191.993 83.517) (end 192.738 84.262) (width 0.2) (layer "F.Cu") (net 20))
 (segment (start 198.232 84.194) (end 198.3 84.126) (width 0.2) (layer "F.Cu") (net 4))
 (segment (start 195.0975 84.194) (end 198.232 84.194) (width 0.2) (layer "F.Cu") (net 4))
 (segment (start 190.768 83.9495) (end 193.5225 86.704) (width 0.2) (layer "F.Cu") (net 24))
 (segment (start 190.644 81.043) (end 190.768 81.043) (width 0.2) (layer "F.Cu") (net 24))
 (segment (start 187.96 78.359) (end 190.644 81.043) (width 0.2) (layer "F.Cu") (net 24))
 (segment (start 190.768 81.043) (end 190.768 83.9495) (width 0.2) (layer "F.Cu") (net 24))
 (segment (start 198.262 86.704) (end 198.3 86.666) (width 0.2) (layer "F.Cu") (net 5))
 (segment (start 195.0975 86.704) (end 198.262 86.704) (width 0.2) (layer "F.Cu") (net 5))
 (segment (start 198.292 89.214) (end 198.3 89.206) (width 0.2) (layer "F.Cu") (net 2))
 (segment (start 195.0975 89.214) (end 198.292 89.214) (width 0.2) (layer "F.Cu") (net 2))
 (segment (start 187.96 82.169) (end 190.768 84.977) (width 0.2) (layer "F.Cu") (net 1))
 (segment (start 190.768 86.4595) (end 193.5225 89.214) (width 0.2) (layer "F.Cu") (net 1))
 (segment (start 190.768 84.977) (end 190.768 86.4595) (width 0.2) (layer "F.Cu") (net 1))
 (segment (start 195.0975 91.724) (end 198.278 91.724) (width 0.2) (layer "F.Cu") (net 6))
 (segment (start 198.278 91.724) (end 198.3 91.746) (width 0.2) (layer "F.Cu") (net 6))
 (segment (start 193.5225 91.541498) (end 193.5225 91.724) (width 0.2) (layer "F.Cu") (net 25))
 (segment (start 187.96 85.978998) (end 193.5225 91.541498) (width 0.2) (layer "F.Cu") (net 25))
 (segment (start 195.0975 94.234) (end 198.248 94.234) (width 0.2) (layer "F.Cu") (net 7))
 (segment (start 198.248 94.234) (end 198.3 94.286) (width 0.2) (layer "F.Cu") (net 7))
 (segment (start 189.077498 89.788998) (end 193.5225 94.234) (width 0.2) (layer "F.Cu") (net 19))
 (segment (start 187.96 89.788998) (end 189.077498 89.788998) (width 0.2) (layer "F.Cu") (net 19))
 (segment (start 195.0975 97.051) (end 198.075 97.051) (width 0.2) (layer "F.Cu") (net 8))
 (segment (start 198.075 97.051) (end 198.3 96.826) (width 0.2) (layer "F.Cu") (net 8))
 (segment (start 187.96 93.599) (end 190.0705 93.599) (width 0.2) (layer "F.Cu") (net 26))
 (segment (start 190.0705 93.599) (end 193.5225 97.051) (width 0.2) (layer "F.Cu") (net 26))
 (segment (start 195.0975 99.561) (end 198.105 99.561) (width 0.2) (layer "F.Cu") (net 9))
 (segment (start 198.105 99.561) (end 198.3 99.366) (width 0.2) (layer "F.Cu") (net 9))
 (segment (start 187.96 97.409) (end 191.3705 97.409) (width 0.2) (layer "F.Cu") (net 27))
 (segment (start 191.3705 97.409) (end 193.5225 99.561) (width 0.2) (layer "F.Cu") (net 27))
 (segment (start 192.6705 101.219) (end 193.5225 102.071) (width 0.2) (layer "F.Cu") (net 28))
 (segment (start 187.96 101.219) (end 192.6705 101.219) (width 0.2) (layer "F.Cu") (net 28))
 (segment (start 198.135 102.071) (end 198.3 101.906) (width 0.2) (layer "F.Cu") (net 10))
 (segment (start 195.0975 102.071) (end 198.135 102.071) (width 0.2) (layer "F.Cu") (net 10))
 (segment (start 198.165 104.581) (end 198.3 104.446) (width 0.2) (layer "F.Cu") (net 11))
 (segment (start 195.0975 104.581) (end 198.165 104.581) (width 0.2) (layer "F.Cu") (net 11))
 (segment (start 187.96 105.029) (end 188.048 105.117) (width 0.2) (layer "F.Cu") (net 29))
 (segment (start 188.048 105.117) (end 189.898 105.117) (width 0.2) (layer "F.Cu") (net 29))
 (segment (start 190.434 104.581) (end 193.5225 104.581) (width 0.2) (layer "F.Cu") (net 29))
 (segment (start 189.898 105.117) (end 190.434 104.581) (width 0.2) (layer "F.Cu") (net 29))
 (segment (start 191.7745 108.839) (end 193.5225 107.091) (width 0.2) (layer "F.Cu") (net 22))
 (segment (start 187.96 108.839) (end 191.7745 108.839) (width 0.2) (layer "F.Cu") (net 22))
 (segment (start 198.195 107.091) (end 198.3 106.986) (width 0.2) (layer "F.Cu") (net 12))
 (segment (start 195.0975 107.091) (end 198.195 107.091) (width 0.2) (layer "F.Cu") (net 12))
 (segment (start 198.225 109.601) (end 198.3 109.526) (width 0.2) (layer "F.Cu") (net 13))
 (segment (start 195.0975 109.601) (end 198.225 109.601) (width 0.2) (layer "F.Cu") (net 13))
 (segment (start 187.96 112.649002) (end 190.474498 112.649002) (width 0.2) (layer "F.Cu") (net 30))
 (segment (start 190.474498 112.649002) (end 193.5225 109.601) (width 0.2) (layer "F.Cu") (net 30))
 (segment (start 187.96 116.459002) (end 189.395998 116.459002) (width 0.2) (layer "F.Cu") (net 21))
 (segment (start 189.395998 116.459002) (end 193.497 112.358) (width 0.2) (layer "F.Cu") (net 21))
 (segment (start 198.008 112.358) (end 198.3 112.066) (width 0.2) (layer "F.Cu") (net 14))
 (segment (start 195.072 112.358) (end 198.008 112.358) (width 0.2) (layer "F.Cu") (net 14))
 (segment (start 188.096 120.269) (end 193.497 114.868) (width 0.2) (layer "F.Cu") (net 31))
 (segment (start 187.96 120.269) (end 188.096 120.269) (width 0.2) (layer "F.Cu") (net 31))
 (segment (start 198.038 114.868) (end 198.3 114.606) (width 0.2) (layer "F.Cu") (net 15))
 (segment (start 195.072 114.868) (end 198.038 114.868) (width 0.2) (layer "F.Cu") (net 15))
 (segment (start 187.96 124.079) (end 187.96 122.915) (width 0.2) (layer "F.Cu") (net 32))
 (segment (start 187.96 122.915) (end 193.497 117.378) (width 0.2) (layer "F.Cu") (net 32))
 (segment (start 198.068 117.378) (end 198.3 117.146) (width 0.2) (layer "F.Cu") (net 16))
 (segment (start 195.072 117.378) (end 198.068 117.378) (width 0.2) (layer "F.Cu") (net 16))
 (segment (start 192.964 119.888) (end 193.497 119.888) (width 0.2) (layer "F.Cu") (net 33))
 (segment (start 187.96 127.759) (end 190.722 124.997) (width 0.2) (layer "F.Cu") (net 33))
 (segment (start 190.722 122.066) (end 190.786 122.066) (width 0.2) (layer "F.Cu") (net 33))
 (segment (start 190.722 124.997) (end 190.722 122.066) (width 0.2) (layer "F.Cu") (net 33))
 (segment (start 187.96 127.889) (end 187.96 127.759) (width 0.2) (layer "F.Cu") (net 33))
 (segment (start 190.786 122.066) (end 192.964 119.888) (width 0.2) (layer "F.Cu") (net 33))
 (segment (start 198.098 119.888) (end 198.3 119.686) (width 0.2) (layer "F.Cu") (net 17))
 (segment (start 195.072 119.888) (end 198.098 119.888) (width 0.2) (layer "F.Cu") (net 17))
 (segment (start 192.1 127.559001) (end 192.1 123.795) (width 0.2) (layer "F.Cu") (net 34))
 (segment (start 187.96 131.699001) (end 192.1 127.559001) (width 0.2) (layer "F.Cu") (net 34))
 (segment (start 192.1 123.795) (end 193.497 122.398) (width 0.2) (layer "F.Cu") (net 34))
 (segment (start 198.128 122.398) (end 198.3 122.226) (width 0.2) (layer "F.Cu") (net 18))
 (segment (start 195.072 122.398) (end 198.128 122.398) (width 0.2) (layer "F.Cu") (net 18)))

